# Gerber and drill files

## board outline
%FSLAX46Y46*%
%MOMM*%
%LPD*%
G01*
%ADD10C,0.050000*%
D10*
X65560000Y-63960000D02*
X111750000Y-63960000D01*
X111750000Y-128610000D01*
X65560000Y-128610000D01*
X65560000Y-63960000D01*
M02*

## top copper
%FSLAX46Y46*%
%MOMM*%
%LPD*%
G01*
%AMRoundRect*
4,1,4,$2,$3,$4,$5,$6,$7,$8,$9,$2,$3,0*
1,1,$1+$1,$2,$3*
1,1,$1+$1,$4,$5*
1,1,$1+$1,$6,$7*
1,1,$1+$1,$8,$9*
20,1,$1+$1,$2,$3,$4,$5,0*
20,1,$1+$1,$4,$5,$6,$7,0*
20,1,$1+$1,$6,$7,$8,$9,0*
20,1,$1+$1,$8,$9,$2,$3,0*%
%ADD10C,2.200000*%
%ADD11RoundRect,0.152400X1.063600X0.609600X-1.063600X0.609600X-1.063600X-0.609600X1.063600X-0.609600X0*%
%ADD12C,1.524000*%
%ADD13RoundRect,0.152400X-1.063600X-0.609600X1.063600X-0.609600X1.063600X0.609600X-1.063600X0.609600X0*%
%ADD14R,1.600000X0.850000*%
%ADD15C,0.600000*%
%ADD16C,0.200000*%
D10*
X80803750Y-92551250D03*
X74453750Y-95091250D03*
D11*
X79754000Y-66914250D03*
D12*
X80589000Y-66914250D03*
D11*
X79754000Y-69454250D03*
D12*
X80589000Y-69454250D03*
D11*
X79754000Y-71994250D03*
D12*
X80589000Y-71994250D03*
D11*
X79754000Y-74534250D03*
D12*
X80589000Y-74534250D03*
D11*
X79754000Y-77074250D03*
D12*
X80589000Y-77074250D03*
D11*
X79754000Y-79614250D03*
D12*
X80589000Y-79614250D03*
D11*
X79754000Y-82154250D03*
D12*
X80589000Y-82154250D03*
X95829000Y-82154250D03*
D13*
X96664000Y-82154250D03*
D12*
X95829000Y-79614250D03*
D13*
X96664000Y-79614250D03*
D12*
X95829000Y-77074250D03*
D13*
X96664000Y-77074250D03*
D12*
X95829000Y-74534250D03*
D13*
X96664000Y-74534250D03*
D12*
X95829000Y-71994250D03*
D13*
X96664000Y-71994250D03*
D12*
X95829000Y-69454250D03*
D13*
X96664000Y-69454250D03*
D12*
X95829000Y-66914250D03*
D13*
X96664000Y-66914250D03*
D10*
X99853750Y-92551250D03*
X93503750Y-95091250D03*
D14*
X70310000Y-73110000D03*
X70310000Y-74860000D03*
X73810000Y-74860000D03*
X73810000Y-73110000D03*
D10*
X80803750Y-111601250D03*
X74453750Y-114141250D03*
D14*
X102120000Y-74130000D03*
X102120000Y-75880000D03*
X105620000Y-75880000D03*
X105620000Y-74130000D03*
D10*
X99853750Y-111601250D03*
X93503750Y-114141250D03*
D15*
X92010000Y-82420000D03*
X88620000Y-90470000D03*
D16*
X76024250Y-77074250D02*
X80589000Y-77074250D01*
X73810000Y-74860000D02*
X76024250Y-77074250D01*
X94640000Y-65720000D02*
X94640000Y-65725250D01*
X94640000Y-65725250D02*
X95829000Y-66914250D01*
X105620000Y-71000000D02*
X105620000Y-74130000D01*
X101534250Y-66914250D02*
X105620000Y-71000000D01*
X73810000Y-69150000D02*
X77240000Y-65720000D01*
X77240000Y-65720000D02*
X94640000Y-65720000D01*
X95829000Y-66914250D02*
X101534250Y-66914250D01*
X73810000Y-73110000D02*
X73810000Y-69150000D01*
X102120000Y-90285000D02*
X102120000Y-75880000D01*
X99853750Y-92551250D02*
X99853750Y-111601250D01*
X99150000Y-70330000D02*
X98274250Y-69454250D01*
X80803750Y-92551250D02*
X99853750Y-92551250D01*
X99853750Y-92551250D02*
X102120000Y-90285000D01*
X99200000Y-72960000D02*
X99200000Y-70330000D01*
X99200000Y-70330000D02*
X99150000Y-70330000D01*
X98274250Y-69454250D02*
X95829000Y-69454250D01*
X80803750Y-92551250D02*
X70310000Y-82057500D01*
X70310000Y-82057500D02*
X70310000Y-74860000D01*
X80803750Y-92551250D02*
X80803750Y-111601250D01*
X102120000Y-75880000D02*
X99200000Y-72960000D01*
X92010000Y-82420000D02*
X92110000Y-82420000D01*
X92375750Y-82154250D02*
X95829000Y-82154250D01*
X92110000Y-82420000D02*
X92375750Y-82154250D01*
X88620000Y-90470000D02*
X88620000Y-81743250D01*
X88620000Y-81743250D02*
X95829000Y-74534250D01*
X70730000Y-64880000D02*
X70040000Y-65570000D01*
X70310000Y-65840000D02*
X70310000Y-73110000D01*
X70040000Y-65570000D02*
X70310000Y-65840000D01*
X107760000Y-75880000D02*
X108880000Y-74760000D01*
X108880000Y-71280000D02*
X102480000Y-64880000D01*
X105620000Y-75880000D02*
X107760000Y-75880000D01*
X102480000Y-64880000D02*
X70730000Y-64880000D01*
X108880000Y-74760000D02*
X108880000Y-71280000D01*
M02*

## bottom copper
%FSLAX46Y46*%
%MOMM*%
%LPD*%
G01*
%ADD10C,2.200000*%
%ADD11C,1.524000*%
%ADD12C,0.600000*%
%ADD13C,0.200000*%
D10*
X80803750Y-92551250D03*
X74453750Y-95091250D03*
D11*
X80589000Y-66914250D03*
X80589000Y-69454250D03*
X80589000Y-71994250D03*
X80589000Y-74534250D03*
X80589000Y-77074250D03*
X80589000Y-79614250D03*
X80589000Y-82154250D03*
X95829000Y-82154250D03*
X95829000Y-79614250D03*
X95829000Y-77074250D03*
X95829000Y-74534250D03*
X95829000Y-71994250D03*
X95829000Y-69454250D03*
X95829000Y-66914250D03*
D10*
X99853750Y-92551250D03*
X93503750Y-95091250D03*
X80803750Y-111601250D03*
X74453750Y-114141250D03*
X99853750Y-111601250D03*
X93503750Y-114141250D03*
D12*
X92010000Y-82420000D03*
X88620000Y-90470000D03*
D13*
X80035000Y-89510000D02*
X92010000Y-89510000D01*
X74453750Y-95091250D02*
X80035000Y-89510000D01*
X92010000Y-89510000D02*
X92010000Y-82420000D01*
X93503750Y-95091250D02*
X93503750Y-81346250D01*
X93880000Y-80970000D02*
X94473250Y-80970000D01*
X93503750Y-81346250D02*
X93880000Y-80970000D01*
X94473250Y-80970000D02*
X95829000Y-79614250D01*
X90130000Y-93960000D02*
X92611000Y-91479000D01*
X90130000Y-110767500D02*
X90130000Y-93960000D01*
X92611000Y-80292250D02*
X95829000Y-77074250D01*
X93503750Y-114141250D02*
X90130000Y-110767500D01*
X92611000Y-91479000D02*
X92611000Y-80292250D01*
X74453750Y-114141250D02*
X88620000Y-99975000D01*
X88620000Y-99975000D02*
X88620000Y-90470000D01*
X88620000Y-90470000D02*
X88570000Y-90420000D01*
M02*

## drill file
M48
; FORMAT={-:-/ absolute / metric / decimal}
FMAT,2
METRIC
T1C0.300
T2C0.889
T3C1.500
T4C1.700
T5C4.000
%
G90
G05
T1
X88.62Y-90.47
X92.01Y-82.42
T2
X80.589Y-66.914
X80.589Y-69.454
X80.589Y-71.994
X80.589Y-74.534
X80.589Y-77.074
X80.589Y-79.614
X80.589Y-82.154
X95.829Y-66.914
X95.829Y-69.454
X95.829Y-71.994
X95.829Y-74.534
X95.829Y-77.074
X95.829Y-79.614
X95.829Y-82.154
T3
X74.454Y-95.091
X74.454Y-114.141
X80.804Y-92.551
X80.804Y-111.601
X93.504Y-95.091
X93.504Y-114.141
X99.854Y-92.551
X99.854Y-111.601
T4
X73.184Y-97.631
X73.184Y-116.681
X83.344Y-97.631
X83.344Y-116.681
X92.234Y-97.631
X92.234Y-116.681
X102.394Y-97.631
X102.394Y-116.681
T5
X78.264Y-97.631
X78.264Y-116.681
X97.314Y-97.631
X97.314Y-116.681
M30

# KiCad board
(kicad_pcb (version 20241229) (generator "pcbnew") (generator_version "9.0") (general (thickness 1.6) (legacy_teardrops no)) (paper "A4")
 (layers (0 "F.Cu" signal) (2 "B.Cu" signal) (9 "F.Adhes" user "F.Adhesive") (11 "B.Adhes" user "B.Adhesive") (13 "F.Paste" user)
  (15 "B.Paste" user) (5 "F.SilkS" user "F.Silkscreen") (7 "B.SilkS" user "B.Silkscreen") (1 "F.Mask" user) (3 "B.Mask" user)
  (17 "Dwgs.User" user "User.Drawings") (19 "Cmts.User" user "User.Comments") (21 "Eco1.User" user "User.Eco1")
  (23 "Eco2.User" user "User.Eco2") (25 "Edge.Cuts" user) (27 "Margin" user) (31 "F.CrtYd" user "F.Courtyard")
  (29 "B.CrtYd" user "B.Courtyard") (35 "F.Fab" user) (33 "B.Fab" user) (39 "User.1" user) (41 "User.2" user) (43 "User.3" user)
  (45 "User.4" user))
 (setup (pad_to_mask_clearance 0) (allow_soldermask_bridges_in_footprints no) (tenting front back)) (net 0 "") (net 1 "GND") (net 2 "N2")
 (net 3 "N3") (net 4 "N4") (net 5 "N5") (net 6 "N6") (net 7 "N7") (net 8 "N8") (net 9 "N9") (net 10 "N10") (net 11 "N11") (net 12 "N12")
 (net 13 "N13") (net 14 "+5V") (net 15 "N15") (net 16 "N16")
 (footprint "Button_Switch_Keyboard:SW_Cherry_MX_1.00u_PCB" (layer "F.Cu") (at 80.80375 92.55125)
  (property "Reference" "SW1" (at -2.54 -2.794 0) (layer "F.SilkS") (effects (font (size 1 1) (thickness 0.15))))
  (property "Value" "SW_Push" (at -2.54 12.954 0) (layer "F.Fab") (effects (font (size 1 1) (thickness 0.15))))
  (pad "" np_thru_hole circle (at -7.62 5.08) (size 1.7 1.7) (drill 1.7) (layers "*.Cu" "*.Mask"))
  (pad "" np_thru_hole circle (at -2.54 5.08) (size 4 4) (drill 4) (layers "*.Cu" "*.Mask"))
  (pad "" np_thru_hole circle (at 2.54 5.08) (size 1.7 1.7) (drill 1.7) (layers "*.Cu" "*.Mask"))
  (pad "1" thru_hole circle (at 0 0) (size 2.2 2.2) (drill 1.5) (layers "*.Cu" "*.Mask") (remove_unused_layers no) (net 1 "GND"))
  (pad "2" thru_hole circle (at -6.35 2.54) (size 2.2 2.2) (drill 1.5) (layers "*.Cu" "*.Mask") (remove_unused_layers no) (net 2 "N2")))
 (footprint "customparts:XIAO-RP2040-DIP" (layer "F.Cu") (at 88.209 74.53425)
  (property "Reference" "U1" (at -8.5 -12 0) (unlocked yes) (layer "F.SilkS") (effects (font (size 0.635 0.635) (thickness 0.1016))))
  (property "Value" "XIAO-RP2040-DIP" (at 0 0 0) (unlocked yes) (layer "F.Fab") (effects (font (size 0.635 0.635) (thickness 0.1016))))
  (pad "1" smd roundrect (at -8.455 -7.62 180) (size 2.432 1.524) (layers "F.Cu" "F.Mask") (roundrect_rratio 0.1) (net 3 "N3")
   (thermal_bridge_angle 45))
  (pad "1" thru_hole circle (at -7.62 -7.62 180) (size 1.524 1.524) (drill 0.889) (layers "*.Cu" "*.Mask") (remove_unused_layers no)
   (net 3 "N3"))
  (pad "2" smd roundrect (at -8.455 -5.08 180) (size 2.432 1.524) (layers "F.Cu" "F.Mask") (roundrect_rratio 0.1) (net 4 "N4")
   (thermal_bridge_angle 45))
  (pad "2" thru_hole circle (at -7.62 -5.08 180) (size 1.524 1.524) (drill 0.889) (layers "*.Cu" "*.Mask") (remove_unused_layers no)
   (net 4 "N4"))
  (pad "3" smd roundrect (at -8.455 -2.54 180) (size 2.432 1.524) (layers "F.Cu" "F.Mask") (roundrect_rratio 0.1) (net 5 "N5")
   (thermal_bridge_angle 45))
  (pad "3" thru_hole circle (at -7.62 -2.54 180) (size 1.524 1.524) (drill 0.889) (layers "*.Cu" "*.Mask") (remove_unused_layers no)
   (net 5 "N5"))
  (pad "4" smd roundrect (at -8.455 0 180) (size 2.432 1.524) (layers "F.Cu" "F.Mask") (roundrect_rratio 0.1) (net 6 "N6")
   (thermal_bridge_angle 45))
  (pad "4" thru_hole circle (at -7.62 0 180) (size 1.524 1.524) (drill 0.889) (layers "*.Cu" "*.Mask") (remove_unused_layers no)
   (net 6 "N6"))
  (pad "5" smd roundrect (at -8.455 2.54 180) (size 2.432 1.524) (layers "F.Cu" "F.Mask") (roundrect_rratio 0.1) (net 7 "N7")
   (thermal_bridge_angle 45))
  (pad "5" thru_hole circle (at -7.62 2.54 180) (size 1.524 1.524) (drill 0.889) (layers "*.Cu" "*.Mask") (remove_unused_layers no)
   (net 7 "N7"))
  (pad "6" smd roundrect (at -8.455 5.08 180) (size 2.432 1.524) (layers "F.Cu" "F.Mask") (roundrect_rratio 0.1) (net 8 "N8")
   (thermal_bridge_angle 45))
  (pad "6" thru_hole circle (at -7.62 5.08 180) (size 1.524 1.524) (drill 0.889) (layers "*.Cu" "*.Mask") (remove_unused_layers no)
   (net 8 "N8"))
  (pad "7" smd roundrect (at -8.455 7.62 180) (size 2.432 1.524) (layers "F.Cu" "F.Mask") (roundrect_rratio 0.1) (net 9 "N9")
   (thermal_bridge_angle 45))
  (pad "7" thru_hole circle (at -7.62 7.62 180) (size 1.524 1.524) (drill 0.889) (layers "*.Cu" "*.Mask") (remove_unused_layers no)
   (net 9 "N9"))
  (pad "8" thru_hole circle (at 7.62 7.62) (size 1.524 1.524) (drill 0.889) (layers "*.Cu" "*.Mask") (remove_unused_layers no) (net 2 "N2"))
  (pad "8" smd roundrect (at 8.455 7.62) (size 2.432 1.524) (layers "F.Cu" "F.Mask") (roundrect_rratio 0.1) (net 2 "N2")
   (thermal_bridge_angle 45))
  (pad "9" thru_hole circle (at 7.62 5.08) (size 1.524 1.524) (drill 0.889) (layers "*.Cu" "*.Mask") (remove_unused_layers no)
   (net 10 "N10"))
  (pad "9" smd roundrect (at 8.455 5.08) (size 2.432 1.524) (layers "F.Cu" "F.Mask") (roundrect_rratio 0.1) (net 10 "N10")
   (thermal_bridge_angle 45))
  (pad "10" thru_hole circle (at 7.62 2.54) (size 1.524 1.524) (drill 0.889) (layers "*.Cu" "*.Mask") (remove_unused_layers no)
   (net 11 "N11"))
  (pad "10" smd roundrect (at 8.455 2.54) (size 2.432 1.524) (layers "F.Cu" "F.Mask") (roundrect_rratio 0.1) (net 11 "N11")
   (thermal_bridge_angle 45))
  (pad "11" thru_hole circle (at 7.62 0) (size 1.524 1.524) (drill 0.889) (layers "*.Cu" "*.Mask") (remove_unused_layers no) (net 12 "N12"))
  (pad "11" smd roundrect (at 8.455 0) (size 2.432 1.524) (layers "F.Cu" "F.Mask") (roundrect_rratio 0.1) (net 12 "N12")
   (thermal_bridge_angle 45))
  (pad "12" thru_hole circle (at 7.62 -2.54) (size 1.524 1.524) (drill 0.889) (layers "*.Cu" "*.Mask") (remove_unused_layers no)
   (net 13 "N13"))
  (pad "12" smd roundrect (at 8.455 -2.54) (size 2.432 1.524) (layers "F.Cu" "F.Mask") (roundrect_rratio 0.1) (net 13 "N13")
   (thermal_bridge_angle 45))
  (pad "13" thru_hole circle (at 7.62 -5.08) (size 1.524 1.524) (drill 0.889) (layers "*.Cu" "*.Mask") (remove_unused_layers no)
   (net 1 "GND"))
  (pad "13" smd roundrect (at 8.455 -5.08) (size 2.432 1.524) (layers "F.Cu" "F.Mask") (roundrect_rratio 0.1) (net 1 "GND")
   (thermal_bridge_angle 45))
  (pad "14" thru_hole circle (at 7.62 -7.62) (size 1.524 1.524) (drill 0.889) (layers "*.Cu" "*.Mask") (remove_unused_layers no)
   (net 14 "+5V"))
  (pad "14" smd roundrect (at 8.455 -7.62) (size 2.432 1.524) (layers "F.Cu" "F.Mask") (roundrect_rratio 0.1) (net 14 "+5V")
   (thermal_bridge_angle 45)))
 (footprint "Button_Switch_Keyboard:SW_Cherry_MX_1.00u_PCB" (layer "F.Cu") (at 99.85375 92.55125)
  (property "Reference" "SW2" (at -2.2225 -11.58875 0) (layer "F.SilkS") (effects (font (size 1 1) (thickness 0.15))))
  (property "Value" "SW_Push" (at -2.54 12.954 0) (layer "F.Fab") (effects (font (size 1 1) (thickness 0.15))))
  (pad "" np_thru_hole circle (at -7.62 5.08) (size 1.7 1.7) (drill 1.7) (layers "*.Cu" "*.Mask"))
  (pad "" np_thru_hole circle (at -2.54 5.08) (size 4 4) (drill 4) (layers "*.Cu" "*.Mask"))
  (pad "" np_thru_hole circle (at 2.54 5.08) (size 1.7 1.7) (drill 1.7) (layers "*.Cu" "*.Mask"))
  (pad "1" thru_hole circle (at 0 0) (size 2.2 2.2) (drill 1.5) (layers "*.Cu" "*.Mask") (remove_unused_layers no) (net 1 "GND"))
  (pad "2" thru_hole circle (at -6.35 2.54) (size 2.2 2.2) (drill 1.5) (layers "*.Cu" "*.Mask") (remove_unused_layers no) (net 10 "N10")))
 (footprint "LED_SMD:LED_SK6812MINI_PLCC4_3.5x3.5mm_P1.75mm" (layer "F.Cu") (at 72.06 73.985)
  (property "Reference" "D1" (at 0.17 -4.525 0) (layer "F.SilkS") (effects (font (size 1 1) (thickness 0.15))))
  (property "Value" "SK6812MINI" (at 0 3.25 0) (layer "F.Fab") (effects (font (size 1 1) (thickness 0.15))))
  (pad "1" smd rect (at -1.75 -0.875) (size 1.6 0.85) (layers "F.Cu" "F.Mask" "F.Paste") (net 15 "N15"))
  (pad "2" smd rect (at -1.75 0.875) (size 1.6 0.85) (layers "F.Cu" "F.Mask" "F.Paste") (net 1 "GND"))
  (pad "3" smd rect (at 1.75 0.875) (size 1.6 0.85) (layers "F.Cu" "F.Mask" "F.Paste") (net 7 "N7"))
  (pad "4" smd rect (at 1.75 -0.875) (size 1.6 0.85) (layers "F.Cu" "F.Mask" "F.Paste") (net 14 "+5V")))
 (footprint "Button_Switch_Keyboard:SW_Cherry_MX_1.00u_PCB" (layer "F.Cu") (at 80.80375 111.60125)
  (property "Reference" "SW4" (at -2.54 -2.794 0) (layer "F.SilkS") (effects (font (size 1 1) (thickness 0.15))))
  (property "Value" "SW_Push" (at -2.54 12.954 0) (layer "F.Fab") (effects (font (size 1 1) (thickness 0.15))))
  (pad "" np_thru_hole circle (at -7.62 5.08) (size 1.7 1.7) (drill 1.7) (layers "*.Cu" "*.Mask"))
  (pad "" np_thru_hole circle (at -2.54 5.08) (size 4 4) (drill 4) (layers "*.Cu" "*.Mask"))
  (pad "" np_thru_hole circle (at 2.54 5.08) (size 1.7 1.7) (drill 1.7) (layers "*.Cu" "*.Mask"))
  (pad "1" thru_hole circle (at 0 0) (size 2.2 2.2) (drill 1.5) (layers "*.Cu" "*.Mask") (remove_unused_layers no) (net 1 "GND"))
  (pad "2" thru_hole circle (at -6.35 2.54) (size 2.2 2.2) (drill 1.5) (layers "*.Cu" "*.Mask") (remove_unused_layers no) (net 12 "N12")))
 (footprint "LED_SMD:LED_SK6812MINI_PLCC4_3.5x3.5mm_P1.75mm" (layer "F.Cu") (at 103.87 75.005)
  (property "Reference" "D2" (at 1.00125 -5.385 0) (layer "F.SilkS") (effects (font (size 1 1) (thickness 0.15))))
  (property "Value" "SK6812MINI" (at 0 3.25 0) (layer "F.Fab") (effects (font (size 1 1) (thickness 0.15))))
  (pad "1" smd rect (at -1.75 -0.875) (size 1.6 0.85) (layers "F.Cu" "F.Mask" "F.Paste") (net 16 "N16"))
  (pad "2" smd rect (at -1.75 0.875) (size 1.6 0.85) (layers "F.Cu" "F.Mask" "F.Paste") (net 1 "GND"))
  (pad "3" smd rect (at 1.75 0.875) (size 1.6 0.85) (layers "F.Cu" "F.Mask" "F.Paste") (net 15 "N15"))
  (pad "4" smd rect (at 1.75 -0.875) (size 1.6 0.85) (layers "F.Cu" "F.Mask" "F.Paste") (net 14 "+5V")))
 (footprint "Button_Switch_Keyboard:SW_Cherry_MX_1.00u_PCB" (layer "F.Cu") (at 99.85375 111.60125)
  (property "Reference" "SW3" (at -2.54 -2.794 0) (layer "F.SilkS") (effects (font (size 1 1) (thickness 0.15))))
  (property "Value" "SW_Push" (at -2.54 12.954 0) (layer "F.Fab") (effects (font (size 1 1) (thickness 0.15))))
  (pad "" np_thru_hole circle (at -7.62 5.08) (size 1.7 1.7) (drill 1.7) (layers "*.Cu" "*.Mask"))
  (pad "" np_thru_hole circle (at -2.54 5.08) (size 4 4) (drill 4) (layers "*.Cu" "*.Mask"))
  (pad "" np_thru_hole circle (at 2.54 5.08) (size 1.7 1.7) (drill 1.7) (layers "*.Cu" "*.Mask"))
  (pad "1" thru_hole circle (at 0 0) (size 2.2 2.2) (drill 1.5) (layers "*.Cu" "*.Mask") (remove_unused_layers no) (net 1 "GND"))
  (pad "2" thru_hole circle (at -6.35 2.54) (size 2.2 2.2) (drill 1.5) (layers "*.Cu" "*.Mask") (remove_unused_layers no) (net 11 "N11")))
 (gr_rect (start 65.56 63.96) (end 111.75 128.61) (stroke (width 0.05) (type default)) (fill no) (layer "Edge.Cuts"))
 (segment (start 76.02425 77.07425) (end 80.589 77.07425) (width 0.2) (layer "F.Cu") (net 7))
 (segment (start 73.81 74.86) (end 76.02425 77.07425) (width 0.2) (layer "F.Cu") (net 7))
 (segment (start 94.64 65.72) (end 94.64 65.72525) (width 0.2) (layer "F.Cu") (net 14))
 (segment (start 94.64 65.72525) (end 95.829 66.91425) (width 0.2) (layer "F.Cu") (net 14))
 (segment (start 105.62 71) (end 105.62 74.13) (width 0.2) (layer "F.Cu") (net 14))
 (segment (start 101.53425 66.91425) (end 105.62 71) (width 0.2) (layer "F.Cu") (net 14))
 (segment (start 73.81 69.15) (end 77.24 65.72) (width 0.2) (layer "F.Cu") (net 14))
 (segment (start 77.24 65.72) (end 94.64 65.72) (width 0.2) (layer "F.Cu") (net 14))
 (segment (start 95.829 66.91425) (end 101.53425 66.91425) (width 0.2) (layer "F.Cu") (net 14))
 (segment (start 73.81 73.11) (end 73.81 69.15) (width 0.2) (layer "F.Cu") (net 14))
 (segment (start 102.12 90.285) (end 102.12 75.88) (width 0.2) (layer "F.Cu") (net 1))
 (segment (start 99.85375 92.55125) (end 99.85375 111.60125) (width 0.2) (layer "F.Cu") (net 1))
 (segment (start 99.15 70.33) (end 98.27425 69.45425) (width 0.2) (layer "F.Cu") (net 1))
 (segment (start 80.80375 92.55125) (end 99.85375 92.55125) (width 0.2) (layer "F.Cu") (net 1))
 (segment (start 99.85375 92.55125) (end 102.12 90.285) (width 0.2) (layer "F.Cu") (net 1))
 (segment (start 99.2 72.96) (end 99.2 70.33) (width 0.2) (layer "F.Cu") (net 1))
 (segment (start 99.2 70.33) (end 99.15 70.33) (width 0.2) (layer "F.Cu") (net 1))
 (segment (start 98.27425 69.45425) (end 95.829 69.45425) (width 0.2) (layer "F.Cu") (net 1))
 (segment (start 80.80375 92.55125) (end 70.31 82.0575) (width 0.2) (layer "F.Cu") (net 1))
 (segment (start 70.31 82.0575) (end 70.31 74.86) (width 0.2) (layer "F.Cu") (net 1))
 (segment (start 80.80375 92.55125) (end 80.80375 111.60125) (width 0.2) (layer "F.Cu") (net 1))
 (segment (start 102.12 75.88) (end 99.2 72.96) (width 0.2) (layer "F.Cu") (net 1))
 (segment (start 92.01 82.42) (end 92.11 82.42) (width 0.2) (layer "F.Cu") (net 2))
 (segment (start 92.37575 82.15425) (end 95.829 82.15425) (width 0.2) (layer "F.Cu") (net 2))
 (segment (start 92.11 82.42) (end 92.37575 82.15425) (width 0.2) (layer "F.Cu") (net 2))
 (via (at 92.01 82.42) (size 0.6) (drill 0.3) (layers "F.Cu" "B.Cu") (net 2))
 (segment (start 80.035 89.51) (end 92.01 89.51) (width 0.2) (layer "B.Cu") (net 2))
 (segment (start 74.45375 95.09125) (end 80.035 89.51) (width 0.2) (layer "B.Cu") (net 2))
 (segment (start 92.01 89.51) (end 92.01 82.42) (width 0.2) (layer "B.Cu") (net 2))
 (segment (start 93.50375 95.09125) (end 93.50375 81.34625) (width 0.2) (layer "B.Cu") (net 10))
 (segment (start 93.88 80.97) (end 94.47325 80.97) (width 0.2) (layer "B.Cu") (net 10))
 (segment (start 93.50375 81.34625) (end 93.88 80.97) (width 0.2) (layer "B.Cu") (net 10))
 (segment (start 94.47325 80.97) (end 95.829 79.61425) (width 0.2) (layer "B.Cu") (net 10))
 (segment (start 90.13 93.96) (end 92.611 91.479) (width 0.2) (layer "B.Cu") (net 11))
 (segment (start 90.13 110.7675) (end 90.13 93.96) (width 0.2) (layer "B.Cu") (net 11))
 (segment (start 92.611 80.29225) (end 95.829 77.07425) (width 0.2) (layer "B.Cu") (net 11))
 (segment (start 93.50375 114.14125) (end 90.13 110.7675) (width 0.2) (layer "B.Cu") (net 11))
 (segment (start 92.611 91.479) (end 92.611 80.29225) (width 0.2) (layer "B.Cu") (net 11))
 (segment (start 88.62 90.47) (end 88.62 81.74325) (width 0.2) (layer "F.Cu") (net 12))
 (segment (start 88.62 81.74325) (end 95.829 74.53425) (width 0.2) (layer "F.Cu") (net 12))
 (via (at 88.62 90.47) (size 0.6) (drill 0.3) (layers "F.Cu" "B.Cu") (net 12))
 (segment (start 74.45375 114.14125) (end 88.62 99.975) (width 0.2) (layer "B.Cu") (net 12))
 (segment (start 88.62 99.975) (end 88.62 90.47) (width 0.2) (layer "B.Cu") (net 12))
 (segment (start 88.62 90.47) (end 88.57 90.42) (width 0.2) (layer "B.Cu") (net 12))
 (segment (start 70.73 64.88) (end 70.04 65.57) (width 0.2) (layer "F.Cu") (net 15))
 (segment (start 70.31 65.84) (end 70.31 73.11) (width 0.2) (layer "F.Cu") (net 15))
 (segment (start 70.04 65.57) (end 70.31 65.84) (width 0.2) (layer "F.Cu") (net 15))
 (segment (start 107.76 75.88) (end 108.88 74.76) (width 0.2) (layer "F.Cu") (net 15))
 (segment (start 108.88 71.28) (end 102.48 64.88) (width 0.2) (layer "F.Cu") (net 15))
 (segment (start 105.62 75.88) (end 107.76 75.88) (width 0.2) (layer "F.Cu") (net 15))
 (segment (start 102.48 64.88) (end 70.73 64.88) (width 0.2) (layer "F.Cu") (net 15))
 (segment (start 108.88 74.76) (end 108.88 71.28) (width 0.2) (layer "F.Cu") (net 15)))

